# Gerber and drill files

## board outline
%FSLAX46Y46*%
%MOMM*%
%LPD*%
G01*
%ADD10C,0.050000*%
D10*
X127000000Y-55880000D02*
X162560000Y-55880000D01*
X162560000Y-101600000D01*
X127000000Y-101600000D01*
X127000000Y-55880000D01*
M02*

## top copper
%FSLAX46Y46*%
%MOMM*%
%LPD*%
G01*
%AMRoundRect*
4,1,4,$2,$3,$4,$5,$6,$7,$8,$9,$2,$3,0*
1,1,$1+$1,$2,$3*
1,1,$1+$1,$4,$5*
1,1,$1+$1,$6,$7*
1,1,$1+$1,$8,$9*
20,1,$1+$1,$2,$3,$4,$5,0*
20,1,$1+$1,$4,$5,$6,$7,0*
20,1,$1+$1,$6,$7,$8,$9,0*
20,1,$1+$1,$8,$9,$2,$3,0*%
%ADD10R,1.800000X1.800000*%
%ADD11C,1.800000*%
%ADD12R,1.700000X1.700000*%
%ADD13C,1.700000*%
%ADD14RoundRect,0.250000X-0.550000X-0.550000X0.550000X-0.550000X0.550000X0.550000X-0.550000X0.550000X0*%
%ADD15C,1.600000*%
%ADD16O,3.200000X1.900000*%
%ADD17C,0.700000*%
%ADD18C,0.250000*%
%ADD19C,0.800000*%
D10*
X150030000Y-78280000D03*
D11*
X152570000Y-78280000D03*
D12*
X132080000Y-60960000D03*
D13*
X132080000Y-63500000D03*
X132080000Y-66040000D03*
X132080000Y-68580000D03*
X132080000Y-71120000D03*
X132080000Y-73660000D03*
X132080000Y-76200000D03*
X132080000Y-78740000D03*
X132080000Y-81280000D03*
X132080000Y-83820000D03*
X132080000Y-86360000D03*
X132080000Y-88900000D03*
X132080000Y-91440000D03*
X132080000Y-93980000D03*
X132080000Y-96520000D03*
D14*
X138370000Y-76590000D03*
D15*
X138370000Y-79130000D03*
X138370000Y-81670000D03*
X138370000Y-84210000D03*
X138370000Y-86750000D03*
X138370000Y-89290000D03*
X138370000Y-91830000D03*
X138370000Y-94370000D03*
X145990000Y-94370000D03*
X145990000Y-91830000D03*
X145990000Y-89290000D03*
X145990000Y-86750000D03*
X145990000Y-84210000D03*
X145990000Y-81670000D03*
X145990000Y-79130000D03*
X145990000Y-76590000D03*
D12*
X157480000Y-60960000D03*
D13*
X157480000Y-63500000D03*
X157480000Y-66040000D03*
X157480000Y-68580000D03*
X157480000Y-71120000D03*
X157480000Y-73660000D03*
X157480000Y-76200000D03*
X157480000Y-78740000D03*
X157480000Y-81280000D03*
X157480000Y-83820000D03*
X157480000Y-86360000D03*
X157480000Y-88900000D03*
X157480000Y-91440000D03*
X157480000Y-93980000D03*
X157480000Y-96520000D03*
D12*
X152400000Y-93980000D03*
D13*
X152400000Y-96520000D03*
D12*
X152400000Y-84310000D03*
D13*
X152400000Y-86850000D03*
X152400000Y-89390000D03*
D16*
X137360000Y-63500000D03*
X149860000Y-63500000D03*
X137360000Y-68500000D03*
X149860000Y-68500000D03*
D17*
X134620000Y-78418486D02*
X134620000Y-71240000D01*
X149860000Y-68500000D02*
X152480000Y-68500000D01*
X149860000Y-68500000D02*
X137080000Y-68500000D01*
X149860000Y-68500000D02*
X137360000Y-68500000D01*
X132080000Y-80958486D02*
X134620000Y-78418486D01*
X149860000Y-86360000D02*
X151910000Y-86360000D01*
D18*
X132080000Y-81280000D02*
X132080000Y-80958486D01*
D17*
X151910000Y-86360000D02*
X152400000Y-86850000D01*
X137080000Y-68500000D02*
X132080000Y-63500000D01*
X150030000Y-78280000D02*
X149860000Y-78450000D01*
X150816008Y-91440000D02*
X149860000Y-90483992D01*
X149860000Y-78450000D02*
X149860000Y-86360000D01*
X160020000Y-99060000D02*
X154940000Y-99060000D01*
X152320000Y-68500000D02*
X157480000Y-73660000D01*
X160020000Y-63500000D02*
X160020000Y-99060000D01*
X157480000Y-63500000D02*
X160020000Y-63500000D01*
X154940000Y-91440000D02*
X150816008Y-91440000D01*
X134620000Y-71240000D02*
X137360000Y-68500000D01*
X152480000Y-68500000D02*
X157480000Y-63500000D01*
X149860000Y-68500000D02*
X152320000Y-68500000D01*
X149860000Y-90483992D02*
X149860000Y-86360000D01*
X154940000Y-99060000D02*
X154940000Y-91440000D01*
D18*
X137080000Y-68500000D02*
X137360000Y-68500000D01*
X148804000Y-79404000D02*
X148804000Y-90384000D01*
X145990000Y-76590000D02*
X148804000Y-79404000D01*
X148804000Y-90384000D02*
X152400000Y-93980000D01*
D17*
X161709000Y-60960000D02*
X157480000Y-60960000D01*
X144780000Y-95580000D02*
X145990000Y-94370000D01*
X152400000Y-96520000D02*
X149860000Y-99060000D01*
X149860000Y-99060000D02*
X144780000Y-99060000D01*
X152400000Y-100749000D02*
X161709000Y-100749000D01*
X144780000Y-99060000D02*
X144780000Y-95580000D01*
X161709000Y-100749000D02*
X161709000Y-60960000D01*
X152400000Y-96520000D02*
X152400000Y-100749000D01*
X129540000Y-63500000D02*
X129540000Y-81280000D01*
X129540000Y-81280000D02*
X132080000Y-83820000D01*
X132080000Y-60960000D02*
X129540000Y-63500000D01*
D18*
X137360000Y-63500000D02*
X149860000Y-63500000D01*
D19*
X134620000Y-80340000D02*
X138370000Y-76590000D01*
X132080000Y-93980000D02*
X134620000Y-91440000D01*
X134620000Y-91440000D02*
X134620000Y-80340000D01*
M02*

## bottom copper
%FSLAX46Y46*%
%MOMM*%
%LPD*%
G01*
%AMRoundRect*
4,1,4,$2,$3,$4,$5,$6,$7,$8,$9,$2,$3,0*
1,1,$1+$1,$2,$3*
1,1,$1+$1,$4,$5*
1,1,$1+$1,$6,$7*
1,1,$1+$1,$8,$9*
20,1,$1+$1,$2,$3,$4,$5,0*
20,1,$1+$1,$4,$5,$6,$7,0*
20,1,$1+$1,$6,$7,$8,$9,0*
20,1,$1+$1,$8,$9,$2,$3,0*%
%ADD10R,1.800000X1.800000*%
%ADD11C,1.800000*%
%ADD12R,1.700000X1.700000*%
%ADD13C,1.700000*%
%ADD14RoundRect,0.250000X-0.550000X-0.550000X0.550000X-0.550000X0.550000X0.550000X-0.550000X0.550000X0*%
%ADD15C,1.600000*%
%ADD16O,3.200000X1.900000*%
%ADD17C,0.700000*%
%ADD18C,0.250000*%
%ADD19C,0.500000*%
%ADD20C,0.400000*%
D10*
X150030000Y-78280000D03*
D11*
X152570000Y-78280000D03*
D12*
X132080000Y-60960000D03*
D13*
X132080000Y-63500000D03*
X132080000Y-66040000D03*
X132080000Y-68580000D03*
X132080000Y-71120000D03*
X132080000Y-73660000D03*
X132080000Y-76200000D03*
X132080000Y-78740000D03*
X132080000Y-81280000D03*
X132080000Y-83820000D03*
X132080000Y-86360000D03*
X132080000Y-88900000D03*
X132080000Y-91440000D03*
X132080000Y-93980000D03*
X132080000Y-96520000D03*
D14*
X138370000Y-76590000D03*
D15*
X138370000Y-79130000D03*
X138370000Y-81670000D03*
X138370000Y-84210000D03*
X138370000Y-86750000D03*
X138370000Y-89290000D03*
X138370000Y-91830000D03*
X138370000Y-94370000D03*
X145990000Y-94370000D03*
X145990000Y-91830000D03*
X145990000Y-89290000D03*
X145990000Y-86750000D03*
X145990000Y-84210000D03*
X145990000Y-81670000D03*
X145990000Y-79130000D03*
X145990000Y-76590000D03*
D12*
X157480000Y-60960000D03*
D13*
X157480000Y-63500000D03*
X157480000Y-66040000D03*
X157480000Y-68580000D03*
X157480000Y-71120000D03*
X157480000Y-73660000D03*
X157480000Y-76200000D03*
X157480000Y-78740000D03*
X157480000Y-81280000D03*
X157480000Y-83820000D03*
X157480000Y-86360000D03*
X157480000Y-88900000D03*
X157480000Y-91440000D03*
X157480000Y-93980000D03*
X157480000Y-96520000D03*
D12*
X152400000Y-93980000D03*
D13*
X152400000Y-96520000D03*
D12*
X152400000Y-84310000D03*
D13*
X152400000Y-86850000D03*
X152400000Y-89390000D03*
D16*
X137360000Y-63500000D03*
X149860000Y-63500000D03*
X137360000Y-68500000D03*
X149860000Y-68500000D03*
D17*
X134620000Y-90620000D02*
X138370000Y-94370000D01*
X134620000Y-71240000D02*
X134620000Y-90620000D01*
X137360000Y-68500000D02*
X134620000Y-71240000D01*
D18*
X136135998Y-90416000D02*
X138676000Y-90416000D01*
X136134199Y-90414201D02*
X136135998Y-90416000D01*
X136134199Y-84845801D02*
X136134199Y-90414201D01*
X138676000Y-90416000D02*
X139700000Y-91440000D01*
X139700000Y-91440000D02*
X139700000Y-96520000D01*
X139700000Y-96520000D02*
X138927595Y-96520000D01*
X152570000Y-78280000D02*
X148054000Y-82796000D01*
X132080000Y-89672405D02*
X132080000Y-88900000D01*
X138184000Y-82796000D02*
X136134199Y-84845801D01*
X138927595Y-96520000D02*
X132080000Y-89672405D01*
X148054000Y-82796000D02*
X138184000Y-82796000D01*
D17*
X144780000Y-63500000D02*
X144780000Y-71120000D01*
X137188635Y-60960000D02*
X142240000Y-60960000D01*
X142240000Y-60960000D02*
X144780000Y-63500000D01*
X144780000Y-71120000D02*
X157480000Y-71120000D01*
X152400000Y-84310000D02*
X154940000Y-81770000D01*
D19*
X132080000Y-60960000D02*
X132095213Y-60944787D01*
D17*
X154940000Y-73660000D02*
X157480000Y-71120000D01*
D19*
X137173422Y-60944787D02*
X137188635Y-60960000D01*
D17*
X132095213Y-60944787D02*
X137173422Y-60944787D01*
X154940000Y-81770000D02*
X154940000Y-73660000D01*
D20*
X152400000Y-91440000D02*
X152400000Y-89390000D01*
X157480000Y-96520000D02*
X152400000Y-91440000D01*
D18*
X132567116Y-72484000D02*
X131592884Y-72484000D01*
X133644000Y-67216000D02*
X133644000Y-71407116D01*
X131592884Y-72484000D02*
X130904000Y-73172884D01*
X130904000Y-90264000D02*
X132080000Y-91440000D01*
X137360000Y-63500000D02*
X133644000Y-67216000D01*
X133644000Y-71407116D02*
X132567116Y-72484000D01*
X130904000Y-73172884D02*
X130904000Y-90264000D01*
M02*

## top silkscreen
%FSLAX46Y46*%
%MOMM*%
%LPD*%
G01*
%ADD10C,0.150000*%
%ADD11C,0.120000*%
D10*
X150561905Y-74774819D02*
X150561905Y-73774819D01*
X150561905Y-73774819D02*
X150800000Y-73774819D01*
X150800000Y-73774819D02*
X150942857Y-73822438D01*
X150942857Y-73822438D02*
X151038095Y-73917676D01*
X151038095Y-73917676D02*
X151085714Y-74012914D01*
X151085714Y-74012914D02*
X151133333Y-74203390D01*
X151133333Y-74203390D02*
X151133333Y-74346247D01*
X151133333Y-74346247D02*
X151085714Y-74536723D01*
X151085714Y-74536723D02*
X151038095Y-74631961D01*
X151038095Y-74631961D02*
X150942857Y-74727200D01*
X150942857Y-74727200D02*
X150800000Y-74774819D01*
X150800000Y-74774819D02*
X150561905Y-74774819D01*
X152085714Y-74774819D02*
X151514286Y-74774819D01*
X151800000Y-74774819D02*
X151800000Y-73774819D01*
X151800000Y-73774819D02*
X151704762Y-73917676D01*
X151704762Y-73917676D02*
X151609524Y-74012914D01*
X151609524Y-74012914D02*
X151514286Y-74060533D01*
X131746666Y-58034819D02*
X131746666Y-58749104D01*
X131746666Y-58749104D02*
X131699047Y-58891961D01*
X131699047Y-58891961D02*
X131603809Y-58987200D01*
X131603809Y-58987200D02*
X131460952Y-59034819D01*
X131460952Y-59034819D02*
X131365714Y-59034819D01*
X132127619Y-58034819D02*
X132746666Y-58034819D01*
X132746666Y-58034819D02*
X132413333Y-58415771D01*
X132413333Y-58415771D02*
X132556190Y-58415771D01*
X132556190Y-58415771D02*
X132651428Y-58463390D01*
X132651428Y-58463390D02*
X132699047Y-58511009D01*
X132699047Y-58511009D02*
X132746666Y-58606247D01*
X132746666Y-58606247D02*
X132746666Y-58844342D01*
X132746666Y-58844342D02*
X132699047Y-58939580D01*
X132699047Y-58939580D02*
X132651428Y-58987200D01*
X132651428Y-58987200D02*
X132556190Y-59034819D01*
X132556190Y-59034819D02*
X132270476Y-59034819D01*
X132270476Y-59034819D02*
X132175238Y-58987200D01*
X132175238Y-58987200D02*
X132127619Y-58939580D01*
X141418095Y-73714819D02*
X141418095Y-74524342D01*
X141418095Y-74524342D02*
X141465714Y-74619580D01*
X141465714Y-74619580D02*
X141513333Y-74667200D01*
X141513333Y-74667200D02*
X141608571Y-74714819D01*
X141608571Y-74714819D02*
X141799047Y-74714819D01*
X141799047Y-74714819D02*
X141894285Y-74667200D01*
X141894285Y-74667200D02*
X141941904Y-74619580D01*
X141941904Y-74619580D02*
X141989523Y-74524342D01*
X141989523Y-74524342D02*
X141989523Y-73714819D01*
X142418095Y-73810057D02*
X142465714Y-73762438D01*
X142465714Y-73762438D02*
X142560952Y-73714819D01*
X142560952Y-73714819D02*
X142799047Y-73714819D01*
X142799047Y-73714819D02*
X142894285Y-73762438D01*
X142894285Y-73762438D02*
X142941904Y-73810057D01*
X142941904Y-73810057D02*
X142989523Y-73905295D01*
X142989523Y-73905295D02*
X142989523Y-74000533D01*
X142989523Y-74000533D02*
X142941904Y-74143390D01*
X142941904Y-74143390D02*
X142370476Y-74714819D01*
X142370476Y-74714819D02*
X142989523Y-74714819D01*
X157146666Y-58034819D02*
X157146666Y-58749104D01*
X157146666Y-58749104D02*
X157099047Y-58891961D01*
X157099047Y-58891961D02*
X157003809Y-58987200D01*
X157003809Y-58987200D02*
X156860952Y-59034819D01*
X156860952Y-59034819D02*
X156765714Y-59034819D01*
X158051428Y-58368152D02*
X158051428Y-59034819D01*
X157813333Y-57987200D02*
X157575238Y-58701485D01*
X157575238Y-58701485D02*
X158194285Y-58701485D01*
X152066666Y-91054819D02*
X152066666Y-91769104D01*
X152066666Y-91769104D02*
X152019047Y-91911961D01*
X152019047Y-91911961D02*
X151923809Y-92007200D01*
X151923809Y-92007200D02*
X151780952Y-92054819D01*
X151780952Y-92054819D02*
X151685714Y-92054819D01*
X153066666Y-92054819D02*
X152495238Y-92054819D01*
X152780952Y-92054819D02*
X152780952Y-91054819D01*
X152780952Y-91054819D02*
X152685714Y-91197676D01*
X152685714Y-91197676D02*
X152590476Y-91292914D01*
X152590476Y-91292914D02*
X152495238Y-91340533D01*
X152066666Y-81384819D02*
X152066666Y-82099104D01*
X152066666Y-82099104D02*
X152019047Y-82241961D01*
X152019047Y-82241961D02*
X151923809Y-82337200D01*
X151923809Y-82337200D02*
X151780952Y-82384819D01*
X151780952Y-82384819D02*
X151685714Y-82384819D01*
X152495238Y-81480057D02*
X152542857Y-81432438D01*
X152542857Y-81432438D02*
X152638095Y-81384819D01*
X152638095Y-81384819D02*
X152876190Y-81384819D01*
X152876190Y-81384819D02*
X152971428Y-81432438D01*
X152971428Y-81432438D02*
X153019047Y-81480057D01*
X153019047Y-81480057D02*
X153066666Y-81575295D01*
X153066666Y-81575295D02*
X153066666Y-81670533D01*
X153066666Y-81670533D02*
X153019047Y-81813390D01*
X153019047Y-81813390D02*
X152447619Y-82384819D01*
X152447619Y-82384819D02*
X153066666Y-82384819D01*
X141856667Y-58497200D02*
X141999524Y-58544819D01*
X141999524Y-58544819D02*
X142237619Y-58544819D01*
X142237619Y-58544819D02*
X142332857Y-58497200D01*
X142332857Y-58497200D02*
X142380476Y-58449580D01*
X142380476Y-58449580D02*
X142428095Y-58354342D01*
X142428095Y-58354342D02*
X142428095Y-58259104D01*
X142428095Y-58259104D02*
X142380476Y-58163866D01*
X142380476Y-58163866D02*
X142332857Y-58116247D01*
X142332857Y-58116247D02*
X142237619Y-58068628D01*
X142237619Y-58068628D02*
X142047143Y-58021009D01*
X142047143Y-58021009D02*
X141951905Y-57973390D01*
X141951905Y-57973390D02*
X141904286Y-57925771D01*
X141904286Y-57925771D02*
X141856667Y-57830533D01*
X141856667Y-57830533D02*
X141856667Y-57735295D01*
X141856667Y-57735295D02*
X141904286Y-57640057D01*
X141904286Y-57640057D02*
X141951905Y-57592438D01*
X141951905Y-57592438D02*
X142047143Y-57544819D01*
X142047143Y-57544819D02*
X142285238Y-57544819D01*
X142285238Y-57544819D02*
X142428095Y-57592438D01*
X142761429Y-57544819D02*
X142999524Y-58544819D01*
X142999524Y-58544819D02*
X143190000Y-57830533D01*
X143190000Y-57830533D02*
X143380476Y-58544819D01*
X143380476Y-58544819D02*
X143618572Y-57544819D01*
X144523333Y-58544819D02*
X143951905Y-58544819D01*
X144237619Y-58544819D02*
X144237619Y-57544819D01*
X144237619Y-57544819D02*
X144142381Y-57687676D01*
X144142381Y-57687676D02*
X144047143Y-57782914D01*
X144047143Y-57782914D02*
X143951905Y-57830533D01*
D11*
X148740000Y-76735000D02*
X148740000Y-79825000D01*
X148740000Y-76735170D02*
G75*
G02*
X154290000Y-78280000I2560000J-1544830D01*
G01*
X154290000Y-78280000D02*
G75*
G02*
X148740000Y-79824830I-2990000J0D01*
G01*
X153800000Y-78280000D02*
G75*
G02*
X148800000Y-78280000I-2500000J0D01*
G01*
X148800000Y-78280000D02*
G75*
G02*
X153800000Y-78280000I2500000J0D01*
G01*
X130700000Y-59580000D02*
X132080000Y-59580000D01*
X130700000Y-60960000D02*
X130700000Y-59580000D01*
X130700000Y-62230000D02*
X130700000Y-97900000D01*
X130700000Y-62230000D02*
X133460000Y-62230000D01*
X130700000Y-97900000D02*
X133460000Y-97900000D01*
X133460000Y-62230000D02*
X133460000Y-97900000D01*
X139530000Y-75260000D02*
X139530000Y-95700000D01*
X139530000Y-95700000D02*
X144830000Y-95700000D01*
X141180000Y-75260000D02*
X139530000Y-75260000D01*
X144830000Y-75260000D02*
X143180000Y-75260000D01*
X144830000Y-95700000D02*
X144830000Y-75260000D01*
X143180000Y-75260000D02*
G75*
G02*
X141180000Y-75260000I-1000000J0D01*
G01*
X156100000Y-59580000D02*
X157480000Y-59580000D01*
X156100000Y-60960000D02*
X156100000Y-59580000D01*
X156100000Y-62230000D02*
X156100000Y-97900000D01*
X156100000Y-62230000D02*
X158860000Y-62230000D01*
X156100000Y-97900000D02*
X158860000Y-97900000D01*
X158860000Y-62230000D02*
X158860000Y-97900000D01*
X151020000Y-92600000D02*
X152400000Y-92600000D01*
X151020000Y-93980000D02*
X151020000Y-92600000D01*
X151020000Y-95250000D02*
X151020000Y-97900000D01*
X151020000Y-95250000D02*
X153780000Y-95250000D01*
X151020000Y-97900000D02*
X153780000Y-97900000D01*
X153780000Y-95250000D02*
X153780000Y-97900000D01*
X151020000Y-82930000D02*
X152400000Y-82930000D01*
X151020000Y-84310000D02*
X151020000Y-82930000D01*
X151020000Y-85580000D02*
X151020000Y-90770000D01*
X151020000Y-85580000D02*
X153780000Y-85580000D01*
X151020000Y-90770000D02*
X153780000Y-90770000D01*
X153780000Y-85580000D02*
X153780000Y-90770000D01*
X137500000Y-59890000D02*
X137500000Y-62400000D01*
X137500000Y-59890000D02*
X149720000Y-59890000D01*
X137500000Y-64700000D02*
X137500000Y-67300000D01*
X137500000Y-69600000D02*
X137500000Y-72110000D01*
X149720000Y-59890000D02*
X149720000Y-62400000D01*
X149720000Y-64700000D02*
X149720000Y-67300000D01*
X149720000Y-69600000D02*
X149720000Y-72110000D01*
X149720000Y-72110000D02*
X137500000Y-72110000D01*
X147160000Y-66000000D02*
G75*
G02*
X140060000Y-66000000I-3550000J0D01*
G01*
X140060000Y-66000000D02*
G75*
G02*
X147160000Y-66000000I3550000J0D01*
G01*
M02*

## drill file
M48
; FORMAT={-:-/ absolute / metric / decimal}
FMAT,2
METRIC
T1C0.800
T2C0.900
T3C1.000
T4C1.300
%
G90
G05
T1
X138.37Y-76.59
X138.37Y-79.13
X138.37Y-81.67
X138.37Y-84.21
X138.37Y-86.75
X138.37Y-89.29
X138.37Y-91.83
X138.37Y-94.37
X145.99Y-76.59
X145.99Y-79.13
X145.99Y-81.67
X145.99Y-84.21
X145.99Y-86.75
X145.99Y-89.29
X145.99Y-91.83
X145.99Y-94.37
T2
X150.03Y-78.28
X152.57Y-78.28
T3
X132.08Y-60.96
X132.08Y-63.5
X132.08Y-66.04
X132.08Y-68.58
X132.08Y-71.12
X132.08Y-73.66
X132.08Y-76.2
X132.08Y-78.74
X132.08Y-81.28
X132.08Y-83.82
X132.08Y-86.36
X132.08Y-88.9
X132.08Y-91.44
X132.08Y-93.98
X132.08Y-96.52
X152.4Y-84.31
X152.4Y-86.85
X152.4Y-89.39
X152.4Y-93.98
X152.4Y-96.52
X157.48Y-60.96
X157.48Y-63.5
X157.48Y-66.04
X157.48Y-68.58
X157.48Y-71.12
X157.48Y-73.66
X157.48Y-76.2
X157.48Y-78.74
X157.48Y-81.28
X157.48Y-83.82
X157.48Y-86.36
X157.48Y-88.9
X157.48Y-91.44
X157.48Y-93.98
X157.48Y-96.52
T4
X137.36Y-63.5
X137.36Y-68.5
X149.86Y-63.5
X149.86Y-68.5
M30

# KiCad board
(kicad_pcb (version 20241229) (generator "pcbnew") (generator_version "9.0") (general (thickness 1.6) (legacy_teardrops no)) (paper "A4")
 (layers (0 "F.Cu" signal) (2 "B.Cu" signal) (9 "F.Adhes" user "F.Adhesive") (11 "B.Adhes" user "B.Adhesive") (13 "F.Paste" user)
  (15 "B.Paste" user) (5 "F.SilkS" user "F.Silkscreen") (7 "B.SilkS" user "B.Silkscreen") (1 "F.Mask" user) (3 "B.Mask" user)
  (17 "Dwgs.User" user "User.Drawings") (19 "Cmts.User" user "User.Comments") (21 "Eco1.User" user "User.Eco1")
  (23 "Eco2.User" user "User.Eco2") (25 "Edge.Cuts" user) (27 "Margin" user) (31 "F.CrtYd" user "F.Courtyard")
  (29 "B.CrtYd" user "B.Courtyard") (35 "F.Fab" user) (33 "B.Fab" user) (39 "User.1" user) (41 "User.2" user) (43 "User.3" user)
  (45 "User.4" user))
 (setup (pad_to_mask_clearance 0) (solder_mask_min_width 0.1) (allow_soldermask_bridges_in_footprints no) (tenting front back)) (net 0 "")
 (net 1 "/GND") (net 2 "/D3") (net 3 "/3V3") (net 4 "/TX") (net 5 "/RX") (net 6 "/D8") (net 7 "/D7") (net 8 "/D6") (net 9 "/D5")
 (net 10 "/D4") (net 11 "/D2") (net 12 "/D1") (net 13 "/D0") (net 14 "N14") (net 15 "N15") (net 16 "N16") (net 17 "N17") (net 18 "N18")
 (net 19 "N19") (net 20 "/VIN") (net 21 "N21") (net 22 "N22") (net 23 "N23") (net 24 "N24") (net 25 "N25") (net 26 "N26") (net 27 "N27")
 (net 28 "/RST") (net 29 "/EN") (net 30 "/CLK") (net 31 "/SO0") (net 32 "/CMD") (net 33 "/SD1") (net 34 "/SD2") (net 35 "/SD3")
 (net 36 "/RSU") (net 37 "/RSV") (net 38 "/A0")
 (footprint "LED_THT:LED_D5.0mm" (layer "F.Cu") (at 150.03 78.28)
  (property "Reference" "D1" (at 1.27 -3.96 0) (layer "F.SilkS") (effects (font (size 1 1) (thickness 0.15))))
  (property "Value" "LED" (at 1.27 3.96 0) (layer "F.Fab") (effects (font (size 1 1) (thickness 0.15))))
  (fp_line (start -1.29 -1.545) (end -1.29 1.545) (stroke (width 0.12) (type solid)) (layer "F.SilkS"))
  (fp_arc (start -1.29 -1.54483) (mid 2.071779 -2.880495) (end 4.26 0) (stroke (width 0.12) (type solid)) (layer "F.SilkS"))
  (fp_arc (start 4.26 0) (mid 2.071779 2.880495) (end -1.29 1.54483) (stroke (width 0.12) (type solid)) (layer "F.SilkS"))
  (fp_circle (center 1.27 0) (end 3.77 0) (stroke (width 0.12) (type solid)) (fill no) (layer "F.SilkS"))
  (pad "1" thru_hole rect (at 0 0) (size 1.8 1.8) (drill 0.9) (layers "*.Cu" "*.Mask") (remove_unused_layers no) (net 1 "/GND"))
  (pad "2" thru_hole circle (at 2.54 0) (size 1.8 1.8) (drill 0.9) (layers "*.Cu" "*.Mask") (remove_unused_layers no) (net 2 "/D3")))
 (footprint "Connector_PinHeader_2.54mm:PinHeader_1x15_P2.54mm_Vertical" (layer "F.Cu") (at 132.08 60.96)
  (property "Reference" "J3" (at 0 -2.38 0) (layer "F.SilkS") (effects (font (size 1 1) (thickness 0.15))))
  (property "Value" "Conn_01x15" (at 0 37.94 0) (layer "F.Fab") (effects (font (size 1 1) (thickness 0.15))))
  (fp_line (start -1.38 -1.38) (end 0 -1.38) (stroke (width 0.12) (type solid)) (layer "F.SilkS"))
  (fp_line (start -1.38 0) (end -1.38 -1.38) (stroke (width 0.12) (type solid)) (layer "F.SilkS"))
  (fp_line (start -1.38 1.27) (end -1.38 36.94) (stroke (width 0.12) (type solid)) (layer "F.SilkS"))
  (fp_line (start -1.38 1.27) (end 1.38 1.27) (stroke (width 0.12) (type solid)) (layer "F.SilkS"))
  (fp_line (start -1.38 36.94) (end 1.38 36.94) (stroke (width 0.12) (type solid)) (layer "F.SilkS"))
  (fp_line (start 1.38 1.27) (end 1.38 36.94) (stroke (width 0.12) (type solid)) (layer "F.SilkS"))
  (pad "1" thru_hole rect (at 0 0) (size 1.7 1.7) (drill 1) (layers "*.Cu" "*.Mask") (remove_unused_layers no) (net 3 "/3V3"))
  (pad "2" thru_hole circle (at 0 2.54) (size 1.7 1.7) (drill 1) (layers "*.Cu" "*.Mask") (remove_unused_layers no) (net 1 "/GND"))
  (pad "3" thru_hole circle (at 0 5.08) (size 1.7 1.7) (drill 1) (layers "*.Cu" "*.Mask") (remove_unused_layers no) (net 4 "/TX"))
  (pad "4" thru_hole circle (at 0 7.62) (size 1.7 1.7) (drill 1) (layers "*.Cu" "*.Mask") (remove_unused_layers no) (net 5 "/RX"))
  (pad "5" thru_hole circle (at 0 10.16) (size 1.7 1.7) (drill 1) (layers "*.Cu" "*.Mask") (remove_unused_layers no) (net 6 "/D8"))
  (pad "6" thru_hole circle (at 0 12.7) (size 1.7 1.7) (drill 1) (layers "*.Cu" "*.Mask") (remove_unused_layers no) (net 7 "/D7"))
  (pad "7" thru_hole circle (at 0 15.24) (size 1.7 1.7) (drill 1) (layers "*.Cu" "*.Mask") (remove_unused_layers no) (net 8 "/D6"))
  (pad "8" thru_hole circle (at 0 17.78) (size 1.7 1.7) (drill 1) (layers "*.Cu" "*.Mask") (remove_unused_layers no) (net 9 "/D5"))
  (pad "9" thru_hole circle (at 0 20.32) (size 1.7 1.7) (drill 1) (layers "*.Cu" "*.Mask") (remove_unused_layers no) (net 1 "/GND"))
  (pad "10" thru_hole circle (at 0 22.86) (size 1.7 1.7) (drill 1) (layers "*.Cu" "*.Mask") (remove_unused_layers no) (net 3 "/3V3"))
  (pad "11" thru_hole circle (at 0 25.4) (size 1.7 1.7) (drill 1) (layers "*.Cu" "*.Mask") (remove_unused_layers no) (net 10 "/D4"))
  (pad "12" thru_hole circle (at 0 27.94) (size 1.7 1.7) (drill 1) (layers "*.Cu" "*.Mask") (remove_unused_layers no) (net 2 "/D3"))
  (pad "13" thru_hole circle (at 0 30.48) (size 1.7 1.7) (drill 1) (layers "*.Cu" "*.Mask") (remove_unused_layers no) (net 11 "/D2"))
  (pad "14" thru_hole circle (at 0 33.02) (size 1.7 1.7) (drill 1) (layers "*.Cu" "*.Mask") (remove_unused_layers no) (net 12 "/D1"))
  (pad "15" thru_hole circle (at 0 35.56) (size 1.7 1.7) (drill 1) (layers "*.Cu" "*.Mask") (remove_unused_layers no) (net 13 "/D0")))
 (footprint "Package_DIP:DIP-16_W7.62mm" (layer "F.Cu") (at 138.37 76.59)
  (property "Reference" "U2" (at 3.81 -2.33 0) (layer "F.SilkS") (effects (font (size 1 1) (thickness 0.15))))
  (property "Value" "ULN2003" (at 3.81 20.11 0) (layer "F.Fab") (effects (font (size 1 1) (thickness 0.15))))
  (fp_line (start 1.16 -1.33) (end 1.16 19.11) (stroke (width 0.12) (type solid)) (layer "F.SilkS"))
  (fp_line (start 1.16 19.11) (end 6.46 19.11) (stroke (width 0.12) (type solid)) (layer "F.SilkS"))
  (fp_line (start 2.81 -1.33) (end 1.16 -1.33) (stroke (width 0.12) (type solid)) (layer "F.SilkS"))
  (fp_line (start 6.46 -1.33) (end 4.81 -1.33) (stroke (width 0.12) (type solid)) (layer "F.SilkS"))
  (fp_line (start 6.46 19.11) (end 6.46 -1.33) (stroke (width 0.12) (type solid)) (layer "F.SilkS"))
  (fp_arc (start 4.81 -1.33) (mid 3.81 -0.33) (end 2.81 -1.33) (stroke (width 0.12) (type solid)) (layer "F.SilkS"))
  (pad "1" thru_hole roundrect (at 0 0) (size 1.6 1.6) (drill 0.8) (layers "*.Cu" "*.Mask") (remove_unused_layers no)
   (roundrect_rratio 0.15625) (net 12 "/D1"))
  (pad "2" thru_hole circle (at 0 2.54) (size 1.6 1.6) (drill 0.8) (layers "*.Cu" "*.Mask") (remove_unused_layers no) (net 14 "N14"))
  (pad "3" thru_hole circle (at 0 5.08) (size 1.6 1.6) (drill 0.8) (layers "*.Cu" "*.Mask") (remove_unused_layers no) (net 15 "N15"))
  (pad "4" thru_hole circle (at 0 7.62) (size 1.6 1.6) (drill 0.8) (layers "*.Cu" "*.Mask") (remove_unused_layers no) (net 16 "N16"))
  (pad "5" thru_hole circle (at 0 10.16) (size 1.6 1.6) (drill 0.8) (layers "*.Cu" "*.Mask") (remove_unused_layers no) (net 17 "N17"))
  (pad "6" thru_hole circle (at 0 12.7) (size 1.6 1.6) (drill 0.8) (layers "*.Cu" "*.Mask") (remove_unused_layers no) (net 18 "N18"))
  (pad "7" thru_hole circle (at 0 15.24) (size 1.6 1.6) (drill 0.8) (layers "*.Cu" "*.Mask") (remove_unused_layers no) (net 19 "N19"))
  (pad "8" thru_hole circle (at 0 17.78) (size 1.6 1.6) (drill 0.8) (layers "*.Cu" "*.Mask") (remove_unused_layers no) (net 1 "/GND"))
  (pad "9" thru_hole circle (at 7.62 17.78) (size 1.6 1.6) (drill 0.8) (layers "*.Cu" "*.Mask") (remove_unused_layers no) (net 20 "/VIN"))
  (pad "10" thru_hole circle (at 7.62 15.24) (size 1.6 1.6) (drill 0.8) (layers "*.Cu" "*.Mask") (remove_unused_layers no) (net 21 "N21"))
  (pad "11" thru_hole circle (at 7.62 12.7) (size 1.6 1.6) (drill 0.8) (layers "*.Cu" "*.Mask") (remove_unused_layers no) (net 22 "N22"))
  (pad "12" thru_hole circle (at 7.62 10.16) (size 1.6 1.6) (drill 0.8) (layers "*.Cu" "*.Mask") (remove_unused_layers no) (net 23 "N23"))
  (pad "13" thru_hole circle (at 7.62 7.62) (size 1.6 1.6) (drill 0.8) (layers "*.Cu" "*.Mask") (remove_unused_layers no) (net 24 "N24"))
  (pad "14" thru_hole circle (at 7.62 5.08) (size 1.6 1.6) (drill 0.8) (layers "*.Cu" "*.Mask") (remove_unused_layers no) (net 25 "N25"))
  (pad "15" thru_hole circle (at 7.62 2.54) (size 1.6 1.6) (drill 0.8) (layers "*.Cu" "*.Mask") (remove_unused_layers no) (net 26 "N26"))
  (pad "16" thru_hole circle (at 7.62 0) (size 1.6 1.6) (drill 0.8) (layers "*.Cu" "*.Mask") (remove_unused_layers no) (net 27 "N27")))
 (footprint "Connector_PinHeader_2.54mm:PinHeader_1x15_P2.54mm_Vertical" (layer "F.Cu") (at 157.48 60.96)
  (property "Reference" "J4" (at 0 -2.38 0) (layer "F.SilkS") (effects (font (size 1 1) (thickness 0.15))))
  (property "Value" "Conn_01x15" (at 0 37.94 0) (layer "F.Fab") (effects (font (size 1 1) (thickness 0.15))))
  (fp_line (start -1.38 -1.38) (end 0 -1.38) (stroke (width 0.12) (type solid)) (layer "F.SilkS"))
  (fp_line (start -1.38 0) (end -1.38 -1.38) (stroke (width 0.12) (type solid)) (layer "F.SilkS"))
  (fp_line (start -1.38 1.27) (end -1.38 36.94) (stroke (width 0.12) (type solid)) (layer "F.SilkS"))
  (fp_line (start -1.38 1.27) (end 1.38 1.27) (stroke (width 0.12) (type solid)) (layer "F.SilkS"))
  (fp_line (start -1.38 36.94) (end 1.38 36.94) (stroke (width 0.12) (type solid)) (layer "F.SilkS"))
  (fp_line (start 1.38 1.27) (end 1.38 36.94) (stroke (width 0.12) (type solid)) (layer "F.SilkS"))
  (pad "1" thru_hole rect (at 0 0) (size 1.7 1.7) (drill 1) (layers "*.Cu" "*.Mask") (remove_unused_layers no) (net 20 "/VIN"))
  (pad "2" thru_hole circle (at 0 2.54) (size 1.7 1.7) (drill 1) (layers "*.Cu" "*.Mask") (remove_unused_layers no) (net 1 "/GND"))
  (pad "3" thru_hole circle (at 0 5.08) (size 1.7 1.7) (drill 1) (layers "*.Cu" "*.Mask") (remove_unused_layers no) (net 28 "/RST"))
  (pad "4" thru_hole circle (at 0 7.62) (size 1.7 1.7) (drill 1) (layers "*.Cu" "*.Mask") (remove_unused_layers no) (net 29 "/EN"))
  (pad "5" thru_hole circle (at 0 10.16) (size 1.7 1.7) (drill 1) (layers "*.Cu" "*.Mask") (remove_unused_layers no) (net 3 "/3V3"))
  (pad "6" thru_hole circle (at 0 12.7) (size 1.7 1.7) (drill 1) (layers "*.Cu" "*.Mask") (remove_unused_layers no) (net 1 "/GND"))
  (pad "7" thru_hole circle (at 0 15.24) (size 1.7 1.7) (drill 1) (layers "*.Cu" "*.Mask") (remove_unused_layers no) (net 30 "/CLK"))
  (pad "8" thru_hole circle (at 0 17.78) (size 1.7 1.7) (drill 1) (layers "*.Cu" "*.Mask") (remove_unused_layers no) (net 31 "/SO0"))
  (pad "9" thru_hole circle (at 0 20.32) (size 1.7 1.7) (drill 1) (layers "*.Cu" "*.Mask") (remove_unused_layers no) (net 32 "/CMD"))
  (pad "10" thru_hole circle (at 0 22.86) (size 1.7 1.7) (drill 1) (layers "*.Cu" "*.Mask") (remove_unused_layers no) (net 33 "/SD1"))
  (pad "11" thru_hole circle (at 0 25.4) (size 1.7 1.7) (drill 1) (layers "*.Cu" "*.Mask") (remove_unused_layers no) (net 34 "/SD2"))
  (pad "12" thru_hole circle (at 0 27.94) (size 1.7 1.7) (drill 1) (layers "*.Cu" "*.Mask") (remove_unused_layers no) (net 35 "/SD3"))
  (pad "13" thru_hole circle (at 0 30.48) (size 1.7 1.7) (drill 1) (layers "*.Cu" "*.Mask") (remove_unused_layers no) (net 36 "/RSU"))
  (pad "14" thru_hole circle (at 0 33.02) (size 1.7 1.7) (drill 1) (layers "*.Cu" "*.Mask") (remove_unused_layers no) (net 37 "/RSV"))
  (pad "15" thru_hole circle (at 0 35.56) (size 1.7 1.7) (drill 1) (layers "*.Cu" "*.Mask") (remove_unused_layers no) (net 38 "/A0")))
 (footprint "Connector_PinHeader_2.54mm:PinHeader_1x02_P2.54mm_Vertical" (layer "F.Cu") (at 152.4 93.98)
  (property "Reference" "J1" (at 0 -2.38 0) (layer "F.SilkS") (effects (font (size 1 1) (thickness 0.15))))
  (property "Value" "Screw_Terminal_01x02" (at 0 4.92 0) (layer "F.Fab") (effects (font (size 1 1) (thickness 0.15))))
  (fp_line (start -1.38 -1.38) (end 0 -1.38) (stroke (width 0.12) (type solid)) (layer "F.SilkS"))
  (fp_line (start -1.38 0) (end -1.38 -1.38) (stroke (width 0.12) (type solid)) (layer "F.SilkS"))
  (fp_line (start -1.38 1.27) (end -1.38 3.92) (stroke (width 0.12) (type solid)) (layer "F.SilkS"))
  (fp_line (start -1.38 1.27) (end 1.38 1.27) (stroke (width 0.12) (type solid)) (layer "F.SilkS"))
  (fp_line (start -1.38 3.92) (end 1.38 3.92) (stroke (width 0.12) (type solid)) (layer "F.SilkS"))
  (fp_line (start 1.38 1.27) (end 1.38 3.92) (stroke (width 0.12) (type solid)) (layer "F.SilkS"))
  (pad "1" thru_hole rect (at 0 0) (size 1.7 1.7) (drill 1) (layers "*.Cu" "*.Mask") (remove_unused_layers no) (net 27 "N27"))
  (pad "2" thru_hole circle (at 0 2.54) (size 1.7 1.7) (drill 1) (layers "*.Cu" "*.Mask") (remove_unused_layers no) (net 20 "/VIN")))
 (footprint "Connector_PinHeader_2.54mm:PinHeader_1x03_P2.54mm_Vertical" (layer "F.Cu") (at 152.4 84.31)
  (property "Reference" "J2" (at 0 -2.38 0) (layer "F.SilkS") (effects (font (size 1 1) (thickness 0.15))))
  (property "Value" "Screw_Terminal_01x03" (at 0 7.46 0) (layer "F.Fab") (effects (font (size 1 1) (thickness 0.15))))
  (fp_line (start -1.38 -1.38) (end 0 -1.38) (stroke (width 0.12) (type solid)) (layer "F.SilkS"))
  (fp_line (start -1.38 0) (end -1.38 -1.38) (stroke (width 0.12) (type solid)) (layer "F.SilkS"))
  (fp_line (start -1.38 1.27) (end -1.38 6.46) (stroke (width 0.12) (type solid)) (layer "F.SilkS"))
  (fp_line (start -1.38 1.27) (end 1.38 1.27) (stroke (width 0.12) (type solid)) (layer "F.SilkS"))
  (fp_line (start -1.38 6.46) (end 1.38 6.46) (stroke (width 0.12) (type solid)) (layer "F.SilkS"))
  (fp_line (start 1.38 1.27) (end 1.38 6.46) (stroke (width 0.12) (type solid)) (layer "F.SilkS"))
  (pad "1" thru_hole rect (at 0 0) (size 1.7 1.7) (drill 1) (layers "*.Cu" "*.Mask") (remove_unused_layers no) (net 3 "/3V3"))
  (pad "2" thru_hole circle (at 0 2.54) (size 1.7 1.7) (drill 1) (layers "*.Cu" "*.Mask") (remove_unused_layers no) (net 1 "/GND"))
  (pad "3" thru_hole circle (at 0 5.08) (size 1.7 1.7) (drill 1) (layers "*.Cu" "*.Mask") (remove_unused_layers no) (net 38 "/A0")))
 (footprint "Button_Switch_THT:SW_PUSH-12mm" (layer "F.Cu") (at 137.36 63.5)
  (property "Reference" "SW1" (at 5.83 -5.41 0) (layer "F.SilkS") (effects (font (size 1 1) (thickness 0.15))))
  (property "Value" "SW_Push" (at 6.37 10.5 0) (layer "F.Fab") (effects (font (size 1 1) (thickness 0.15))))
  (fp_line (start 0.14 -3.61) (end 0.14 -1.1) (stroke (width 0.12) (type default)) (layer "F.SilkS"))
  (fp_line (start 0.14 -3.61) (end 12.36 -3.61) (stroke (width 0.12) (type default)) (layer "F.SilkS"))
  (fp_line (start 0.14 1.2) (end 0.14 3.8) (stroke (width 0.12) (type default)) (layer "F.SilkS"))
  (fp_line (start 0.14 6.1) (end 0.14 8.61) (stroke (width 0.12) (type default)) (layer "F.SilkS"))
  (fp_line (start 12.36 -3.61) (end 12.36 -1.1) (stroke (width 0.12) (type default)) (layer "F.SilkS"))
  (fp_line (start 12.36 1.2) (end 12.36 3.8) (stroke (width 0.12) (type default)) (layer "F.SilkS"))
  (fp_line (start 12.36 6.1) (end 12.36 8.61) (stroke (width 0.12) (type default)) (layer "F.SilkS"))
  (fp_line (start 12.36 8.61) (end 0.14 8.61) (stroke (width 0.12) (type default)) (layer "F.SilkS"))
  (fp_circle (center 6.25 2.5) (end 9.8 2.5) (stroke (width 0.12) (type default)) (fill no) (layer "F.SilkS"))
  (pad "1" thru_hole oval (at 0 0) (size 3.2 1.9) (drill 1.3) (layers "*.Cu" "*.Mask") (remove_unused_layers no) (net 11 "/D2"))
  (pad "1" thru_hole oval (at 12.5 0) (size 3.2 1.9) (drill 1.3) (layers "*.Cu" "*.Mask") (remove_unused_layers no) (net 11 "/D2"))
  (pad "2" thru_hole oval (at 0 5) (size 3.2 1.9) (drill 1.3) (layers "*.Cu" "*.Mask") (remove_unused_layers no) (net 1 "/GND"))
  (pad "2" thru_hole oval (at 12.5 5) (size 3.2 1.9) (drill 1.3) (layers "*.Cu" "*.Mask") (remove_unused_layers no) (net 1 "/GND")))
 (gr_rect (start 127 55.88) (end 162.56 101.6) (stroke (width 0.05) (type default)) (fill no) (layer "Edge.Cuts"))
 (segment (start 134.62 78.418486) (end 134.62 71.24) (width 0.7) (layer "F.Cu") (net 1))
 (segment (start 149.86 68.5) (end 152.48 68.5) (width 0.7) (layer "F.Cu") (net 1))
 (segment (start 149.86 68.5) (end 137.08 68.5) (width 0.7) (layer "F.Cu") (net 1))
 (segment (start 149.86 68.5) (end 137.36 68.5) (width 0.7) (layer "F.Cu") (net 1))
 (segment (start 132.08 80.958486) (end 134.62 78.418486) (width 0.7) (layer "F.Cu") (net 1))
 (segment (start 149.86 86.36) (end 151.91 86.36) (width 0.7) (layer "F.Cu") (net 1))
 (segment (start 132.08 81.28) (end 132.08 80.958486) (width 0.25) (layer "F.Cu") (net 1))
 (segment (start 151.91 86.36) (end 152.4 86.85) (width 0.7) (layer "F.Cu") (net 1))
 (segment (start 137.08 68.5) (end 132.08 63.5) (width 0.7) (layer "F.Cu") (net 1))
 (segment (start 150.03 78.28) (end 149.86 78.45) (width 0.7) (layer "F.Cu") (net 1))
 (segment (start 150.816008 91.44) (end 149.86 90.483992) (width 0.7) (layer "F.Cu") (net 1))
 (segment (start 149.86 78.45) (end 149.86 86.36) (width 0.7) (layer "F.Cu") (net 1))
 (segment (start 160.02 99.06) (end 154.94 99.06) (width 0.7) (layer "F.Cu") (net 1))
 (segment (start 152.32 68.5) (end 157.48 73.66) (width 0.7) (layer "F.Cu") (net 1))
 (segment (start 160.02 63.5) (end 160.02 99.06) (width 0.7) (layer "F.Cu") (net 1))
 (segment (start 157.48 63.5) (end 160.02 63.5) (width 0.7) (layer "F.Cu") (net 1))
 (segment (start 154.94 91.44) (end 150.816008 91.44) (width 0.7) (layer "F.Cu") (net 1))
 (segment (start 134.62 71.24) (end 137.36 68.5) (width 0.7) (layer "F.Cu") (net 1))
 (segment (start 152.48 68.5) (end 157.48 63.5) (width 0.7) (layer "F.Cu") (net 1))
 (segment (start 149.86 68.5) (end 152.32 68.5) (width 0.7) (layer "F.Cu") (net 1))
 (segment (start 149.86 90.483992) (end 149.86 86.36) (width 0.7) (layer "F.Cu") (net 1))
 (segment (start 154.94 99.06) (end 154.94 91.44) (width 0.7) (layer "F.Cu") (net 1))
 (segment (start 137.08 68.5) (end 137.36 68.5) (width 0.25) (layer "F.Cu") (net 1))
 (segment (start 134.62 90.62) (end 138.37 94.37) (width 0.7) (layer "B.Cu") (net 1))
 (segment (start 134.62 71.24) (end 134.62 90.62) (width 0.7) (layer "B.Cu") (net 1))
 (segment (start 137.36 68.5) (end 134.62 71.24) (width 0.7) (layer "B.Cu") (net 1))
 (segment (start 136.135998 90.416) (end 138.676 90.416) (width 0.25) (layer "B.Cu") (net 2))
 (segment (start 136.134199 90.414201) (end 136.135998 90.416) (width 0.25) (layer "B.Cu") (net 2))
 (segment (start 136.134199 84.845801) (end 136.134199 90.414201) (width 0.25) (layer "B.Cu") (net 2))
 (segment (start 138.676 90.416) (end 139.7 91.44) (width 0.25) (layer "B.Cu") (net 2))
 (segment (start 139.7 91.44) (end 139.7 96.52) (width 0.25) (layer "B.Cu") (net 2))
 (segment (start 139.7 96.52) (end 138.927595 96.52) (width 0.25) (layer "B.Cu") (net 2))
 (segment (start 152.57 78.28) (end 148.054 82.796) (width 0.25) (layer "B.Cu") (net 2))
 (segment (start 132.08 89.672405) (end 132.08 88.9) (width 0.25) (layer "B.Cu") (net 2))
 (segment (start 138.184 82.796) (end 136.134199 84.845801) (width 0.25) (layer "B.Cu") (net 2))
 (segment (start 138.927595 96.52) (end 132.08 89.672405) (width 0.25) (layer "B.Cu") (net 2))
 (segment (start 148.054 82.796) (end 138.184 82.796) (width 0.25) (layer "B.Cu") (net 2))
 (segment (start 148.804 79.404) (end 148.804 90.384) (width 0.25) (layer "F.Cu") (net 27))
 (segment (start 145.99 76.59) (end 148.804 79.404) (width 0.25) (layer "F.Cu") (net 27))
 (segment (start 148.804 90.384) (end 152.4 93.98) (width 0.25) (layer "F.Cu") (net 27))
 (segment (start 161.709 60.96) (end 157.48 60.96) (width 0.7) (layer "F.Cu") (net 20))
 (segment (start 144.78 95.58) (end 145.99 94.37) (width 0.7) (layer "F.Cu") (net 20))
 (segment (start 152.4 96.52) (end 149.86 99.06) (width 0.7) (layer "F.Cu") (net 20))
 (segment (start 149.86 99.06) (end 144.78 99.06) (width 0.7) (layer "F.Cu") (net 20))
 (segment (start 152.4 100.749) (end 161.709 100.749) (width 0.7) (layer "F.Cu") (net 20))
 (segment (start 144.78 99.06) (end 144.78 95.58) (width 0.7) (layer "F.Cu") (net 20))
 (segment (start 161.709 100.749) (end 161.709 60.96) (width 0.7) (layer "F.Cu") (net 20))
 (segment (start 152.4 96.52) (end 152.4 100.749) (width 0.7) (layer "F.Cu") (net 20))
 (segment (start 129.54 63.5) (end 129.54 81.28) (width 0.7) (layer "F.Cu") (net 3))
 (segment (start 129.54 81.28) (end 132.08 83.82) (width 0.7) (layer "F.Cu") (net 3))
 (segment (start 132.08 60.96) (end 129.54 63.5) (width 0.7) (layer "F.Cu") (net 3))
 (segment (start 144.78 63.5) (end 144.78 71.12) (width 0.7) (layer "B.Cu") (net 3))
 (segment (start 137.188635 60.96) (end 142.24 60.96) (width 0.7) (layer "B.Cu") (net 3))
 (segment (start 142.24 60.96) (end 144.78 63.5) (width 0.7) (layer "B.Cu") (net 3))
 (segment (start 144.78 71.12) (end 157.48 71.12) (width 0.7) (layer "B.Cu") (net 3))
 (segment (start 152.4 84.31) (end 154.94 81.77) (width 0.7) (layer "B.Cu") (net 3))
 (segment (start 132.08 60.96) (end 132.095213 60.944787) (width 0.5) (layer "B.Cu") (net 3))
 (segment (start 154.94 73.66) (end 157.48 71.12) (width 0.7) (layer "B.Cu") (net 3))
 (segment (start 137.173422 60.944787) (end 137.188635 60.96) (width 0.5) (layer "B.Cu") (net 3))
 (segment (start 132.095213 60.944787) (end 137.173422 60.944787) (width 0.7) (layer "B.Cu") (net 3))
 (segment (start 154.94 81.77) (end 154.94 73.66) (width 0.7) (layer "B.Cu") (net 3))
 (segment (start 152.4 91.44) (end 152.4 89.39) (width 0.4) (layer "B.Cu") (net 38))
 (segment (start 157.48 96.52) (end 152.4 91.44) (width 0.4) (layer "B.Cu") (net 38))
 (segment (start 137.36 63.5) (end 149.86 63.5) (width 0.25) (layer "F.Cu") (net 11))
 (segment (start 132.567116 72.484) (end 131.592884 72.484) (width 0.25) (layer "B.Cu") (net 11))
 (segment (start 133.644 67.216) (end 133.644 71.407116) (width 0.25) (layer "B.Cu") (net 11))
 (segment (start 131.592884 72.484) (end 130.904 73.172884) (width 0.25) (layer "B.Cu") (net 11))
 (segment (start 130.904 90.264) (end 132.08 91.44) (width 0.25) (layer "B.Cu") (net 11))
 (segment (start 137.36 63.5) (end 133.644 67.216) (width 0.25) (layer "B.Cu") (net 11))
 (segment (start 133.644 71.407116) (end 132.567116 72.484) (width 0.25) (layer "B.Cu") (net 11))
 (segment (start 130.904 73.172884) (end 130.904 90.264) (width 0.25) (layer "B.Cu") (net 11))
 (segment (start 134.62 80.34) (end 138.37 76.59) (width 0.8) (layer "F.Cu") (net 12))
 (segment (start 132.08 93.98) (end 134.62 91.44) (width 0.8) (layer "F.Cu") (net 12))
 (segment (start 134.62 91.44) (end 134.62 80.34) (width 0.8) (layer "F.Cu") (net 12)))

